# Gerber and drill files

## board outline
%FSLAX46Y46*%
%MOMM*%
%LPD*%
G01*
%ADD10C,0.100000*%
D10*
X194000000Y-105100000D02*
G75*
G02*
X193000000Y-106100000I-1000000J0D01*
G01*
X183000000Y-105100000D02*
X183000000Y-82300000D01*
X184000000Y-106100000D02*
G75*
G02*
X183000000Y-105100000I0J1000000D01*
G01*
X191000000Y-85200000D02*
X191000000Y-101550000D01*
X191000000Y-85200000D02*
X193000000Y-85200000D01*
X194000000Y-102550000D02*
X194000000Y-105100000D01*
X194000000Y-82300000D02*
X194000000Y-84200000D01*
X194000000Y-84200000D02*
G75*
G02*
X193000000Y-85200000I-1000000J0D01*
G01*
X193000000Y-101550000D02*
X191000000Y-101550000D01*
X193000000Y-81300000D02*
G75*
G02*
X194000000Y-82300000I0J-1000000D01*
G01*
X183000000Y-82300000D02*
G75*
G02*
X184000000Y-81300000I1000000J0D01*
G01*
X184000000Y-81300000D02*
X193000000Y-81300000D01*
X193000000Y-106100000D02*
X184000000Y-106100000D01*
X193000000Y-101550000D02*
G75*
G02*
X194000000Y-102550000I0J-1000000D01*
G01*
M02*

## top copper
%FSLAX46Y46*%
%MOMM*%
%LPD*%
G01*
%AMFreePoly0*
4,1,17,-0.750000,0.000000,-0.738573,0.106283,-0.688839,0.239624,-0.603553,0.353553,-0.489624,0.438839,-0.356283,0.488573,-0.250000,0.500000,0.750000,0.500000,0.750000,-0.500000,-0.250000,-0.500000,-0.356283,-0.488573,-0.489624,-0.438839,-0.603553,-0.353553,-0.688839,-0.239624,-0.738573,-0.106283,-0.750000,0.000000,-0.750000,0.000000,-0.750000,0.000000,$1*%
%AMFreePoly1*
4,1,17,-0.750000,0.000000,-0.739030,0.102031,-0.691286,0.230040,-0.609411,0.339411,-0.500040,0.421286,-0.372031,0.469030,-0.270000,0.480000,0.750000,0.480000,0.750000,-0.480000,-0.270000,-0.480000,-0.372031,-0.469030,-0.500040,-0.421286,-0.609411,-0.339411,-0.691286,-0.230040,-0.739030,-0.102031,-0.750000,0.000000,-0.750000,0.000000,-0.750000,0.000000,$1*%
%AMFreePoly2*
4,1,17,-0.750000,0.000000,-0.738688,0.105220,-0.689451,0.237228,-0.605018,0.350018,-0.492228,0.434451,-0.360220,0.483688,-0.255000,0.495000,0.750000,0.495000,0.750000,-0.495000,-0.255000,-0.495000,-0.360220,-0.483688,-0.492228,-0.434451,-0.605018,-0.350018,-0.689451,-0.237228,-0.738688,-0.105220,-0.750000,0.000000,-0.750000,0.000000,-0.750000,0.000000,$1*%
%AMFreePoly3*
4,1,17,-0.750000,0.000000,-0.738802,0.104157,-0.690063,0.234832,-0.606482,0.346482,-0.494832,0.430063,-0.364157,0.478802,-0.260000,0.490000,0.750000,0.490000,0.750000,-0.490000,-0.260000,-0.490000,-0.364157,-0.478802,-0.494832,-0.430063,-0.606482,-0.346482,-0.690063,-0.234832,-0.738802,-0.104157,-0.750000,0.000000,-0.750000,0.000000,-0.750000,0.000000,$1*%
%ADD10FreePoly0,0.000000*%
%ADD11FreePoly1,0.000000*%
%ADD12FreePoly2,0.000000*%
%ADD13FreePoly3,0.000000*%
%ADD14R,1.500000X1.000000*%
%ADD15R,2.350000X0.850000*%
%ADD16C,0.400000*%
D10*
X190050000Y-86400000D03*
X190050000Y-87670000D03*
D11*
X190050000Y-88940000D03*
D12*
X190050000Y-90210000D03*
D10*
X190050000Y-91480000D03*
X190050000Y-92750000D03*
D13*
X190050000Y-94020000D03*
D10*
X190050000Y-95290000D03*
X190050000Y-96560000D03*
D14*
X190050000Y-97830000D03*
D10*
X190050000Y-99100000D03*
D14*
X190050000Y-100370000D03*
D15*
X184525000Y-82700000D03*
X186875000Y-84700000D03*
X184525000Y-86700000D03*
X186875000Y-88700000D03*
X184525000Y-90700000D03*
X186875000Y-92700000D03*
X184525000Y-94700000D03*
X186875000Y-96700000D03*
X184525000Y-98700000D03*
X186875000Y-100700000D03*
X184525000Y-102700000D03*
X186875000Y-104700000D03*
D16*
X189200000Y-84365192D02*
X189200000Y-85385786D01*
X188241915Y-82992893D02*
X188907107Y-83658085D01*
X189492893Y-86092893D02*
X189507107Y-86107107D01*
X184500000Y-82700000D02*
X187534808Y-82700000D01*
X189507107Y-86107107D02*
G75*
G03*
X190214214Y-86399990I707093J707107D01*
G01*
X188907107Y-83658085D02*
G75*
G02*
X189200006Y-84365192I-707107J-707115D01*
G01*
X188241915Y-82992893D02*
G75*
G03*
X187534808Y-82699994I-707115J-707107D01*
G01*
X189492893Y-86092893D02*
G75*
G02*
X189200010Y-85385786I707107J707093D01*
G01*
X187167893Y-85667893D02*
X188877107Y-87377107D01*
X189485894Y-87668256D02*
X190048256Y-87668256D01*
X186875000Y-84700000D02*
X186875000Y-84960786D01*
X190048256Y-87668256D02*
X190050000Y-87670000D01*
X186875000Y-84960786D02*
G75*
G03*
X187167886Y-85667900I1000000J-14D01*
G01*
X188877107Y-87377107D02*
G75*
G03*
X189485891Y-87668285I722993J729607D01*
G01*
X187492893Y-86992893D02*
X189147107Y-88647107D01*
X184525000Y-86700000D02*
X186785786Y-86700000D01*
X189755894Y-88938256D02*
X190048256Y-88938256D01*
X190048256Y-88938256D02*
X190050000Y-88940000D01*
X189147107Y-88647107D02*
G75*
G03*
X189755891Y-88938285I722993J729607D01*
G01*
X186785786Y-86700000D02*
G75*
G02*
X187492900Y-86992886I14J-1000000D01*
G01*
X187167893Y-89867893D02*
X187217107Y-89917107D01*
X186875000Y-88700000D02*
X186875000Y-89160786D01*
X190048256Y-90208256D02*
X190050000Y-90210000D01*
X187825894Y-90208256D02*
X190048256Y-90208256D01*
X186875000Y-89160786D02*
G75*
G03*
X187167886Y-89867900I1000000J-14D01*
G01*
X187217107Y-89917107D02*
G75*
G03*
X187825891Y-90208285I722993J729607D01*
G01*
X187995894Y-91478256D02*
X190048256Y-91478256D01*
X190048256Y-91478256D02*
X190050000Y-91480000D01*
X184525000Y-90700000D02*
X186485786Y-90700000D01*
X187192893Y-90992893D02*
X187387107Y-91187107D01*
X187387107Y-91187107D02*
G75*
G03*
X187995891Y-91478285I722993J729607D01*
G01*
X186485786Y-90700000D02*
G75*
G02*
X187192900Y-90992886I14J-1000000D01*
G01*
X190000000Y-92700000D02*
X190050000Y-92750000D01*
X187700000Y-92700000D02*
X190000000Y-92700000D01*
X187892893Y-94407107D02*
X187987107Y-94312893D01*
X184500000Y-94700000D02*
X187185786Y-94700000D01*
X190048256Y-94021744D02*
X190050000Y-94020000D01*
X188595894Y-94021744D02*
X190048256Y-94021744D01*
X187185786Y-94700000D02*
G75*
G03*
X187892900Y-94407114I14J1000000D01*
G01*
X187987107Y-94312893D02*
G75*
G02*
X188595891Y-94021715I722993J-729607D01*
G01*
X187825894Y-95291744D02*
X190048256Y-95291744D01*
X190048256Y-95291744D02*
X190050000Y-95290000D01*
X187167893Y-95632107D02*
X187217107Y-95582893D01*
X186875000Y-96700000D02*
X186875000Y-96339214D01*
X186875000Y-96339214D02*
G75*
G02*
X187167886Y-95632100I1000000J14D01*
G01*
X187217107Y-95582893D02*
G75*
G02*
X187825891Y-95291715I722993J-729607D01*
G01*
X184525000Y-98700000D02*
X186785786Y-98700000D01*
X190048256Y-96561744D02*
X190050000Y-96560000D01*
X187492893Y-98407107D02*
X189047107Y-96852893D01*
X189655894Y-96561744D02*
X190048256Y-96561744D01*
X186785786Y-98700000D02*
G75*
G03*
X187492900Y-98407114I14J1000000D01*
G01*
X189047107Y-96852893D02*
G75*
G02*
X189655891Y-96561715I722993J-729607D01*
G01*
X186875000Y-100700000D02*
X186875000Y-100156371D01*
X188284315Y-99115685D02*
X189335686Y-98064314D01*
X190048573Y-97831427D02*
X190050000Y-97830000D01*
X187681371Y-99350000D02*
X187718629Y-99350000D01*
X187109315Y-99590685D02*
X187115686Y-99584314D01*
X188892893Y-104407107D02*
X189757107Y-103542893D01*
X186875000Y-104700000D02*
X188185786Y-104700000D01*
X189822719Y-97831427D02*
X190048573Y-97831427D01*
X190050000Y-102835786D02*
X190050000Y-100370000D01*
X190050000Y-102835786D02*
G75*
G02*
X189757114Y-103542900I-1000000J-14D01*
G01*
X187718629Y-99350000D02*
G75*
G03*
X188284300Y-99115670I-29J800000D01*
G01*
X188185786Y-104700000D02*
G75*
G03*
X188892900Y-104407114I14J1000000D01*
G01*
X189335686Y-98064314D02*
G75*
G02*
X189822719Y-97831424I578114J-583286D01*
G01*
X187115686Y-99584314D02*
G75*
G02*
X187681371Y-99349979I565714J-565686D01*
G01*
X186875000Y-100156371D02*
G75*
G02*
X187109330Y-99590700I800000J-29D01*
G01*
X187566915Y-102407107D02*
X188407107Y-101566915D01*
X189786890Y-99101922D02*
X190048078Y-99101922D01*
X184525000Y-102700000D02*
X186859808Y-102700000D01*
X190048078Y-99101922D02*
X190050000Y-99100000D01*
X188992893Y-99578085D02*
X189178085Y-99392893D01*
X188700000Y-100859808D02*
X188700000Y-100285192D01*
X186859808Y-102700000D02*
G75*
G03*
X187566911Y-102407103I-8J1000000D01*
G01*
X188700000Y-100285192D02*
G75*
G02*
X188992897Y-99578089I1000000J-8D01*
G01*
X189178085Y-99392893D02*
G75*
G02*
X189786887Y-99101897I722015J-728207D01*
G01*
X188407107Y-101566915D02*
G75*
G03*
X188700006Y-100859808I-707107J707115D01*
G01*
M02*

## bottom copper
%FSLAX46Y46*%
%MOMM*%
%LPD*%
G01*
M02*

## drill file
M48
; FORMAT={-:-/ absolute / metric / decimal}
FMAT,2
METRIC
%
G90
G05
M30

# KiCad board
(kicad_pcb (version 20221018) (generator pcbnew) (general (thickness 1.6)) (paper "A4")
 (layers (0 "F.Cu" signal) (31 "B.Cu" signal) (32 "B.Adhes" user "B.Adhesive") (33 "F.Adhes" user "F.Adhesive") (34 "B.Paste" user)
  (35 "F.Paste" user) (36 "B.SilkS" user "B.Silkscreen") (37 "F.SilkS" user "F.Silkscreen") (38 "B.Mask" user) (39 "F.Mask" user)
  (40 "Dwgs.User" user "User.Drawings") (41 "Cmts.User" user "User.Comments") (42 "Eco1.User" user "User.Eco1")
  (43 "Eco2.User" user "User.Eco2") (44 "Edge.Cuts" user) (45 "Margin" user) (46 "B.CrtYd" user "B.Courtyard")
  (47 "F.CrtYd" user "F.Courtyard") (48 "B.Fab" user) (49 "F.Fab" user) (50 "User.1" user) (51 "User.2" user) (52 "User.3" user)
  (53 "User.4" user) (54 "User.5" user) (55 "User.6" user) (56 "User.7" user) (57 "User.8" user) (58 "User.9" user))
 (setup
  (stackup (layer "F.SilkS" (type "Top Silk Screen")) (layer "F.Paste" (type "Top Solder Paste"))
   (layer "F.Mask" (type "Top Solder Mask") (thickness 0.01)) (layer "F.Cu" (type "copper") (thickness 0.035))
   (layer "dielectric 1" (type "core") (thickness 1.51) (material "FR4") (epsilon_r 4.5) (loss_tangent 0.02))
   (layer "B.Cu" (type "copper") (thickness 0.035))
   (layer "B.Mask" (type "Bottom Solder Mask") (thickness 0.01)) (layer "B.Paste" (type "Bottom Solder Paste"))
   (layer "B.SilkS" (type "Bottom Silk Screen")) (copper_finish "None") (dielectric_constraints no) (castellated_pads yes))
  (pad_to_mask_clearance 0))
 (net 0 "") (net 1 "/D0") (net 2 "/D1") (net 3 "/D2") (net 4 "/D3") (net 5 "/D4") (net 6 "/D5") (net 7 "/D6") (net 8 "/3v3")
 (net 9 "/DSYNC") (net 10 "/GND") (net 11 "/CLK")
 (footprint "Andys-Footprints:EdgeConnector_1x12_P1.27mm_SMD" (layer "F.Cu") (at 190.8 86.4)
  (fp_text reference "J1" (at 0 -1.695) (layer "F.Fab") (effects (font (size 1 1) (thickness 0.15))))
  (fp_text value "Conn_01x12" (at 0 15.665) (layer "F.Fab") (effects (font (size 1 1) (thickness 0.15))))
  (pad "1" smd roundrect (at -0.75 0) (size 1.5 1) (layers "F.Cu" "F.Paste" "F.Mask") (roundrect_rratio 0.5) (chamfer_ratio 0)
   (chamfer top_right bottom_right) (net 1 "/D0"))
  (pad "2" smd roundrect (at -0.75 1.27) (size 1.5 1) (layers "F.Cu" "F.Paste" "F.Mask") (roundrect_rratio 0.5) (chamfer_ratio 0)
   (chamfer top_right bottom_right) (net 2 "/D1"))
  (pad "3" smd roundrect (at -0.75 2.54) (size 1.5 0.96) (layers "F.Cu" "F.Paste" "F.Mask") (roundrect_rratio 0.5) (chamfer_ratio 0)
   (chamfer top_right bottom_right) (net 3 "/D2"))
  (pad "4" smd roundrect (at -0.75 3.81) (size 1.5 0.99) (layers "F.Cu" "F.Paste" "F.Mask") (roundrect_rratio 0.5) (chamfer_ratio 0)
   (chamfer top_right bottom_right) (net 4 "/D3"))
  (pad "5" smd roundrect (at -0.75 5.08) (size 1.5 1) (layers "F.Cu" "F.Paste" "F.Mask") (roundrect_rratio 0.5) (chamfer_ratio 0)
   (chamfer top_right bottom_right) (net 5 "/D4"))
  (pad "6" smd roundrect (at -0.75 6.35) (size 1.5 1) (layers "F.Cu" "F.Paste" "F.Mask") (roundrect_rratio 0.5) (chamfer_ratio 0)
   (chamfer top_right bottom_right) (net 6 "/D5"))
  (pad "7" smd roundrect (at -0.75 7.62) (size 1.5 0.98) (layers "F.Cu" "F.Paste" "F.Mask") (roundrect_rratio 0.5) (chamfer_ratio 0)
   (chamfer top_right bottom_right) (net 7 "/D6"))
  (pad "8" smd roundrect (at -0.75 8.89) (size 1.5 1) (layers "F.Cu" "F.Paste" "F.Mask") (roundrect_rratio 0.5) (chamfer_ratio 0)
   (chamfer top_right bottom_right) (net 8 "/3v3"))
  (pad "9" smd roundrect (at -0.75 10.16) (size 1.5 1) (layers "F.Cu" "F.Paste" "F.Mask") (roundrect_rratio 0.5) (chamfer_ratio 0)
   (chamfer top_right bottom_right) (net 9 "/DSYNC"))
  (pad "10" smd rect (at -0.75 11.43) (size 1.5 1) (layers "F.Cu" "F.Paste" "F.Mask") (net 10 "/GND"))
  (pad "11" smd roundrect (at -0.75 12.7) (size 1.5 1) (layers "F.Cu" "F.Paste" "F.Mask") (roundrect_rratio 0.5) (chamfer_ratio 0)
   (chamfer top_right bottom_right) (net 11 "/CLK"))
  (pad "12" smd rect (at -0.75 13.97) (size 1.5 1) (layers "F.Cu" "F.Paste" "F.Mask") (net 10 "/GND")))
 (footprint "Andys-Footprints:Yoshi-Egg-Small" (layer "F.Cu") (at 191.7 103.8)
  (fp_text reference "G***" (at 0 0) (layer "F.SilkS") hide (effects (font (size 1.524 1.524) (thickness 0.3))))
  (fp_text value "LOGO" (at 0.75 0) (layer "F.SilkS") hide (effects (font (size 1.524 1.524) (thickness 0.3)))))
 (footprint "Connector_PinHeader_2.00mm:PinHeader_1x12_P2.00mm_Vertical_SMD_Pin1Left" (layer "F.Cu") (at 185.7 93.7)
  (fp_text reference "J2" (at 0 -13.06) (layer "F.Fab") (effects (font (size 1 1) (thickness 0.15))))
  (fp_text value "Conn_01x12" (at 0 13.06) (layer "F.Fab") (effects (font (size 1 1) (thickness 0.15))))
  (pad "1" smd rect (at -1.175 -11) (size 2.35 0.85) (layers "F.Cu" "F.Paste" "F.Mask") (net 1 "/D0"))
  (pad "2" smd rect (at 1.175 -9) (size 2.35 0.85) (layers "F.Cu" "F.Paste" "F.Mask") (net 2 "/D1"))
  (pad "3" smd rect (at -1.175 -7) (size 2.35 0.85) (layers "F.Cu" "F.Paste" "F.Mask") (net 3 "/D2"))
  (pad "4" smd rect (at 1.175 -5) (size 2.35 0.85) (layers "F.Cu" "F.Paste" "F.Mask") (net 4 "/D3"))
  (pad "5" smd rect (at -1.175 -3) (size 2.35 0.85) (layers "F.Cu" "F.Paste" "F.Mask") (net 5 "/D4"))
  (pad "6" smd rect (at 1.175 -1) (size 2.35 0.85) (layers "F.Cu" "F.Paste" "F.Mask") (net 6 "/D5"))
  (pad "7" smd rect (at -1.175 1) (size 2.35 0.85) (layers "F.Cu" "F.Paste" "F.Mask") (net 7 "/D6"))
  (pad "8" smd rect (at 1.175 3) (size 2.35 0.85) (layers "F.Cu" "F.Paste" "F.Mask") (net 8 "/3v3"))
  (pad "9" smd rect (at -1.175 5) (size 2.35 0.85) (layers "F.Cu" "F.Paste" "F.Mask") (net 9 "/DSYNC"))
  (pad "10" smd rect (at 1.175 7) (size 2.35 0.85) (layers "F.Cu" "F.Paste" "F.Mask") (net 10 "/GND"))
  (pad "11" smd rect (at -1.175 9) (size 2.35 0.85) (layers "F.Cu" "F.Paste" "F.Mask") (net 11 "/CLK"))
  (pad "12" smd rect (at 1.175 11) (size 2.35 0.85) (layers "F.Cu" "F.Paste" "F.Mask") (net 10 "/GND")))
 (gr_arc (start 194 105.1) (mid 193.707107 105.807107) (end 193 106.1) (stroke (width 0.1) (type solid)) (layer "Edge.Cuts"))
 (gr_line (start 183 105.1) (end 183 82.3) (stroke (width 0.1) (type solid)) (layer "Edge.Cuts"))
 (gr_arc (start 184 106.1) (mid 183.292893 105.807107) (end 183 105.1) (stroke (width 0.1) (type solid)) (layer "Edge.Cuts"))
 (gr_line (start 191 85.2) (end 191 101.55) (stroke (width 0.1) (type solid)) (layer "Edge.Cuts"))
 (gr_line (start 191 85.2) (end 193 85.2) (stroke (width 0.1) (type solid)) (layer "Edge.Cuts"))
 (gr_line (start 194 102.55) (end 194 105.1) (stroke (width 0.1) (type solid)) (layer "Edge.Cuts"))
 (gr_line (start 194 82.3) (end 194 84.2) (stroke (width 0.1) (type solid)) (layer "Edge.Cuts"))
 (gr_arc (start 194 84.2) (mid 193.707107 84.907107) (end 193 85.2) (stroke (width 0.1) (type solid)) (layer "Edge.Cuts"))
 (gr_line (start 193 101.55) (end 191 101.55) (stroke (width 0.1) (type solid)) (layer "Edge.Cuts"))
 (gr_arc (start 193 81.3) (mid 193.707107 81.592893) (end 194 82.3) (stroke (width 0.1) (type solid)) (layer "Edge.Cuts"))
 (gr_arc (start 183 82.3) (mid 183.292893 81.592893) (end 184 81.3) (stroke (width 0.1) (type solid)) (layer "Edge.Cuts"))
 (gr_line (start 184 81.3) (end 193 81.3) (stroke (width 0.1) (type solid)) (layer "Edge.Cuts"))
 (gr_line (start 193 106.1) (end 184 106.1) (stroke (width 0.1) (type solid)) (layer "Edge.Cuts"))
 (gr_arc (start 193 101.55) (mid 193.707107 101.842893) (end 194 102.55) (stroke (width 0.1) (type solid)) (layer "Edge.Cuts"))
 (segment (start 189.2 84.365192) (end 189.2 85.385786) (width 0.4) (layer "F.Cu") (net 1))
 (segment (start 188.241915 82.992893) (end 188.907107 83.658085) (width 0.4) (layer "F.Cu") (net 1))
 (segment (start 189.492893 86.092893) (end 189.507107 86.107107) (width 0.4) (layer "F.Cu") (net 1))
 (segment (start 184.5 82.7) (end 187.534808 82.7) (width 0.4) (layer "F.Cu") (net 1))
 (arc (start 189.507107 86.107107) (mid 189.83153 86.32388) (end 190.214214 86.4) (width 0.4) (layer "F.Cu") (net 1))
 (arc (start 188.907107 83.658085) (mid 189.12388 83.982508) (end 189.2 84.365192) (width 0.4) (layer "F.Cu") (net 1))
 (arc (start 188.241915 82.992893) (mid 187.917492 82.77612) (end 187.534808 82.7) (width 0.4) (layer "F.Cu") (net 1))
 (arc (start 189.492893 86.092893) (mid 189.27612 85.76847) (end 189.2 85.385786) (width 0.4) (layer "F.Cu") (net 1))
 (segment (start 187.167893 85.667893) (end 188.877107 87.377107) (width 0.4) (layer "F.Cu") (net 2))
 (segment (start 189.485894 87.668256) (end 190.048256 87.668256) (width 0.4) (layer "F.Cu") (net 2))
 (segment (start 186.875 84.7) (end 186.875 84.960786) (width 0.4) (layer "F.Cu") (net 2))
 (segment (start 190.048256 87.668256) (end 190.05 87.67) (width 0.4) (layer "F.Cu") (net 2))
 (arc (start 186.875 84.960786) (mid 186.95112 85.343469) (end 187.167893 85.667893) (width 0.4) (layer "F.Cu") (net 2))
 (arc (start 188.877107 87.377107) (mid 189.15666 87.573986) (end 189.485894 87.668256) (width 0.4) (layer "F.Cu") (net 2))
 (segment (start 187.492893 86.992893) (end 189.147107 88.647107) (width 0.4) (layer "F.Cu") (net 3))
 (segment (start 184.525 86.7) (end 186.785786 86.7) (width 0.4) (layer "F.Cu") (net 3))
 (segment (start 189.755894 88.938256) (end 190.048256 88.938256) (width 0.4) (layer "F.Cu") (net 3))
 (segment (start 190.048256 88.938256) (end 190.05 88.94) (width 0.4) (layer "F.Cu") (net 3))
 (arc (start 189.147107 88.647107) (mid 189.42666 88.843986) (end 189.755894 88.938256) (width 0.4) (layer "F.Cu") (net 3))
 (arc (start 186.785786 86.7) (mid 187.16847 86.77612) (end 187.492893 86.992893) (width 0.4) (layer "F.Cu") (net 3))
 (segment (start 187.167893 89.867893) (end 187.217107 89.917107) (width 0.4) (layer "F.Cu") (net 4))
 (segment (start 186.875 88.7) (end 186.875 89.160786) (width 0.4) (layer "F.Cu") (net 4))
 (segment (start 190.048256 90.208256) (end 190.05 90.21) (width 0.4) (layer "F.Cu") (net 4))
 (segment (start 187.825894 90.208256) (end 190.048256 90.208256) (width 0.4) (layer "F.Cu") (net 4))
 (arc (start 186.875 89.160786) (mid 186.95112 89.543469) (end 187.167893 89.867893) (width 0.4) (layer "F.Cu") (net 4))
 (arc (start 187.217107 89.917107) (mid 187.49666 90.113986) (end 187.825894 90.208256) (width 0.4) (layer "F.Cu") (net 4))
 (segment (start 187.995894 91.478256) (end 190.048256 91.478256) (width 0.4) (layer "F.Cu") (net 5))
 (segment (start 190.048256 91.478256) (end 190.05 91.48) (width 0.4) (layer "F.Cu") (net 5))
 (segment (start 184.525 90.7) (end 186.485786 90.7) (width 0.4) (layer "F.Cu") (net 5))
 (segment (start 187.192893 90.992893) (end 187.387107 91.187107) (width 0.4) (layer "F.Cu") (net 5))
 (arc (start 187.387107 91.187107) (mid 187.66666 91.383986) (end 187.995894 91.478256) (width 0.4) (layer "F.Cu") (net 5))
 (arc (start 186.485786 90.7) (mid 186.868469 90.77612) (end 187.192893 90.992893) (width 0.4) (layer "F.Cu") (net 5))
 (segment (start 190 92.7) (end 190.05 92.75) (width 0.4) (layer "F.Cu") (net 6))
 (segment (start 187.7 92.7) (end 190 92.7) (width 0.4) (layer "F.Cu") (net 6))
 (segment (start 187.892893 94.407107) (end 187.987107 94.312893) (width 0.4) (layer "F.Cu") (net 7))
 (segment (start 184.5 94.7) (end 187.185786 94.7) (width 0.4) (layer "F.Cu") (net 7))
 (segment (start 190.048256 94.021744) (end 190.05 94.02) (width 0.4) (layer "F.Cu") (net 7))
 (segment (start 188.595894 94.021744) (end 190.048256 94.021744) (width 0.4) (layer "F.Cu") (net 7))
 (arc (start 187.185786 94.7) (mid 187.568469 94.62388) (end 187.892893 94.407107) (width 0.4) (layer "F.Cu") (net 7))
 (arc (start 187.987107 94.312893) (mid 188.26666 94.116014) (end 188.595894 94.021744) (width 0.4) (layer "F.Cu") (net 7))
 (segment (start 187.825894 95.291744) (end 190.048256 95.291744) (width 0.4) (layer "F.Cu") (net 8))
 (segment (start 190.048256 95.291744) (end 190.05 95.29) (width 0.4) (layer "F.Cu") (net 8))
 (segment (start 187.167893 95.632107) (end 187.217107 95.582893) (width 0.4) (layer "F.Cu") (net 8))
 (segment (start 186.875 96.7) (end 186.875 96.339214) (width 0.4) (layer "F.Cu") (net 8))
 (arc (start 186.875 96.339214) (mid 186.95112 95.95653) (end 187.167893 95.632107) (width 0.4) (layer "F.Cu") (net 8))
 (arc (start 187.217107 95.582893) (mid 187.49666 95.386014) (end 187.825894 95.291744) (width 0.4) (layer "F.Cu") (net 8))
 (segment (start 184.525 98.7) (end 186.785786 98.7) (width 0.4) (layer "F.Cu") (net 9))
 (segment (start 190.048256 96.561744) (end 190.05 96.56) (width 0.4) (layer "F.Cu") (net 9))
 (segment (start 187.492893 98.407107) (end 189.047107 96.852893) (width 0.4) (layer "F.Cu") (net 9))
 (segment (start 189.655894 96.561744) (end 190.048256 96.561744) (width 0.4) (layer "F.Cu") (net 9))
 (arc (start 186.785786 98.7) (mid 187.168469 98.62388) (end 187.492893 98.407107) (width 0.4) (layer "F.Cu") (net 9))
 (arc (start 189.047107 96.852893) (mid 189.32666 96.656014) (end 189.655894 96.561744) (width 0.4) (layer "F.Cu") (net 9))
 (segment (start 186.875 100.7) (end 186.875 100.156371) (width 0.4) (layer "F.Cu") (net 10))
 (segment (start 188.284315 99.115685) (end 189.335686 98.064314) (width 0.4) (layer "F.Cu") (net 10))
 (segment (start 190.048573 97.831427) (end 190.05 97.83) (width 0.4) (layer "F.Cu") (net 10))
 (segment (start 187.681371 99.35) (end 187.718629 99.35) (width 0.4) (layer "F.Cu") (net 10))
 (segment (start 187.109315 99.590685) (end 187.115686 99.584314) (width 0.4) (layer "F.Cu") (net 10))
 (segment (start 188.892893 104.407107) (end 189.757107 103.542893) (width 0.4) (layer "F.Cu") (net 10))
 (segment (start 186.875 104.7) (end 188.185786 104.7) (width 0.4) (layer "F.Cu") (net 10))
 (segment (start 189.822719 97.831427) (end 190.048573 97.831427) (width 0.4) (layer "F.Cu") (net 10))
 (segment (start 190.05 102.835786) (end 190.05 100.37) (width 0.4) (layer "F.Cu") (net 10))
 (arc (start 190.05 102.835786) (mid 189.97388 103.218469) (end 189.757107 103.542893) (width 0.4) (layer "F.Cu") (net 10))
 (arc (start 187.718629 99.35) (mid 188.024776 99.289103) (end 188.284315 99.115685) (width 0.4) (layer "F.Cu") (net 10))
 (arc (start 188.185786 104.7) (mid 188.568469 104.62388) (end 188.892893 104.407107) (width 0.4) (layer "F.Cu") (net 10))
 (arc (start 189.335686 98.064314) (mid 189.559325 97.9068) (end 189.822719 97.831427) (width 0.4) (layer "F.Cu") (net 10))
 (arc (start 187.115686 99.584314) (mid 187.375225 99.410896) (end 187.681371 99.35) (width 0.4) (layer "F.Cu") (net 10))
 (arc (start 186.875 100.156371) (mid 186.935897 99.850224) (end 187.109315 99.590685) (width 0.4) (layer "F.Cu") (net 10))
 (segment (start 187.566915 102.407107) (end 188.407107 101.566915) (width 0.4) (layer "F.Cu") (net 11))
 (segment (start 189.78689 99.101922) (end 190.048078 99.101922) (width 0.4) (layer "F.Cu") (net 11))
 (segment (start 184.525 102.7) (end 186.859808 102.7) (width 0.4) (layer "F.Cu") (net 11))
 (segment (start 190.048078 99.101922) (end 190.05 99.1) (width 0.4) (layer "F.Cu") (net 11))
 (segment (start 188.992893 99.578085) (end 189.178085 99.392893) (width 0.4) (layer "F.Cu") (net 11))
 (segment (start 188.7 100.859808) (end 188.7 100.285192) (width 0.4) (layer "F.Cu") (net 11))
 (arc (start 186.859808 102.7) (mid 187.242492 102.62388) (end 187.566915 102.407107) (width 0.4) (layer "F.Cu") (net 11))
 (arc (start 188.7 100.285192) (mid 188.77612 99.902509) (end 188.992893 99.578085) (width 0.4) (layer "F.Cu") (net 11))
 (arc (start 189.178085 99.392893) (mid 189.457636 99.196008) (end 189.78689 99.101922) (width 0.4) (layer "F.Cu") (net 11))
 (arc (start 188.407107 101.566915) (mid 188.62388 101.242492) (end 188.7 100.859808) (width 0.4) (layer "F.Cu") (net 11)))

